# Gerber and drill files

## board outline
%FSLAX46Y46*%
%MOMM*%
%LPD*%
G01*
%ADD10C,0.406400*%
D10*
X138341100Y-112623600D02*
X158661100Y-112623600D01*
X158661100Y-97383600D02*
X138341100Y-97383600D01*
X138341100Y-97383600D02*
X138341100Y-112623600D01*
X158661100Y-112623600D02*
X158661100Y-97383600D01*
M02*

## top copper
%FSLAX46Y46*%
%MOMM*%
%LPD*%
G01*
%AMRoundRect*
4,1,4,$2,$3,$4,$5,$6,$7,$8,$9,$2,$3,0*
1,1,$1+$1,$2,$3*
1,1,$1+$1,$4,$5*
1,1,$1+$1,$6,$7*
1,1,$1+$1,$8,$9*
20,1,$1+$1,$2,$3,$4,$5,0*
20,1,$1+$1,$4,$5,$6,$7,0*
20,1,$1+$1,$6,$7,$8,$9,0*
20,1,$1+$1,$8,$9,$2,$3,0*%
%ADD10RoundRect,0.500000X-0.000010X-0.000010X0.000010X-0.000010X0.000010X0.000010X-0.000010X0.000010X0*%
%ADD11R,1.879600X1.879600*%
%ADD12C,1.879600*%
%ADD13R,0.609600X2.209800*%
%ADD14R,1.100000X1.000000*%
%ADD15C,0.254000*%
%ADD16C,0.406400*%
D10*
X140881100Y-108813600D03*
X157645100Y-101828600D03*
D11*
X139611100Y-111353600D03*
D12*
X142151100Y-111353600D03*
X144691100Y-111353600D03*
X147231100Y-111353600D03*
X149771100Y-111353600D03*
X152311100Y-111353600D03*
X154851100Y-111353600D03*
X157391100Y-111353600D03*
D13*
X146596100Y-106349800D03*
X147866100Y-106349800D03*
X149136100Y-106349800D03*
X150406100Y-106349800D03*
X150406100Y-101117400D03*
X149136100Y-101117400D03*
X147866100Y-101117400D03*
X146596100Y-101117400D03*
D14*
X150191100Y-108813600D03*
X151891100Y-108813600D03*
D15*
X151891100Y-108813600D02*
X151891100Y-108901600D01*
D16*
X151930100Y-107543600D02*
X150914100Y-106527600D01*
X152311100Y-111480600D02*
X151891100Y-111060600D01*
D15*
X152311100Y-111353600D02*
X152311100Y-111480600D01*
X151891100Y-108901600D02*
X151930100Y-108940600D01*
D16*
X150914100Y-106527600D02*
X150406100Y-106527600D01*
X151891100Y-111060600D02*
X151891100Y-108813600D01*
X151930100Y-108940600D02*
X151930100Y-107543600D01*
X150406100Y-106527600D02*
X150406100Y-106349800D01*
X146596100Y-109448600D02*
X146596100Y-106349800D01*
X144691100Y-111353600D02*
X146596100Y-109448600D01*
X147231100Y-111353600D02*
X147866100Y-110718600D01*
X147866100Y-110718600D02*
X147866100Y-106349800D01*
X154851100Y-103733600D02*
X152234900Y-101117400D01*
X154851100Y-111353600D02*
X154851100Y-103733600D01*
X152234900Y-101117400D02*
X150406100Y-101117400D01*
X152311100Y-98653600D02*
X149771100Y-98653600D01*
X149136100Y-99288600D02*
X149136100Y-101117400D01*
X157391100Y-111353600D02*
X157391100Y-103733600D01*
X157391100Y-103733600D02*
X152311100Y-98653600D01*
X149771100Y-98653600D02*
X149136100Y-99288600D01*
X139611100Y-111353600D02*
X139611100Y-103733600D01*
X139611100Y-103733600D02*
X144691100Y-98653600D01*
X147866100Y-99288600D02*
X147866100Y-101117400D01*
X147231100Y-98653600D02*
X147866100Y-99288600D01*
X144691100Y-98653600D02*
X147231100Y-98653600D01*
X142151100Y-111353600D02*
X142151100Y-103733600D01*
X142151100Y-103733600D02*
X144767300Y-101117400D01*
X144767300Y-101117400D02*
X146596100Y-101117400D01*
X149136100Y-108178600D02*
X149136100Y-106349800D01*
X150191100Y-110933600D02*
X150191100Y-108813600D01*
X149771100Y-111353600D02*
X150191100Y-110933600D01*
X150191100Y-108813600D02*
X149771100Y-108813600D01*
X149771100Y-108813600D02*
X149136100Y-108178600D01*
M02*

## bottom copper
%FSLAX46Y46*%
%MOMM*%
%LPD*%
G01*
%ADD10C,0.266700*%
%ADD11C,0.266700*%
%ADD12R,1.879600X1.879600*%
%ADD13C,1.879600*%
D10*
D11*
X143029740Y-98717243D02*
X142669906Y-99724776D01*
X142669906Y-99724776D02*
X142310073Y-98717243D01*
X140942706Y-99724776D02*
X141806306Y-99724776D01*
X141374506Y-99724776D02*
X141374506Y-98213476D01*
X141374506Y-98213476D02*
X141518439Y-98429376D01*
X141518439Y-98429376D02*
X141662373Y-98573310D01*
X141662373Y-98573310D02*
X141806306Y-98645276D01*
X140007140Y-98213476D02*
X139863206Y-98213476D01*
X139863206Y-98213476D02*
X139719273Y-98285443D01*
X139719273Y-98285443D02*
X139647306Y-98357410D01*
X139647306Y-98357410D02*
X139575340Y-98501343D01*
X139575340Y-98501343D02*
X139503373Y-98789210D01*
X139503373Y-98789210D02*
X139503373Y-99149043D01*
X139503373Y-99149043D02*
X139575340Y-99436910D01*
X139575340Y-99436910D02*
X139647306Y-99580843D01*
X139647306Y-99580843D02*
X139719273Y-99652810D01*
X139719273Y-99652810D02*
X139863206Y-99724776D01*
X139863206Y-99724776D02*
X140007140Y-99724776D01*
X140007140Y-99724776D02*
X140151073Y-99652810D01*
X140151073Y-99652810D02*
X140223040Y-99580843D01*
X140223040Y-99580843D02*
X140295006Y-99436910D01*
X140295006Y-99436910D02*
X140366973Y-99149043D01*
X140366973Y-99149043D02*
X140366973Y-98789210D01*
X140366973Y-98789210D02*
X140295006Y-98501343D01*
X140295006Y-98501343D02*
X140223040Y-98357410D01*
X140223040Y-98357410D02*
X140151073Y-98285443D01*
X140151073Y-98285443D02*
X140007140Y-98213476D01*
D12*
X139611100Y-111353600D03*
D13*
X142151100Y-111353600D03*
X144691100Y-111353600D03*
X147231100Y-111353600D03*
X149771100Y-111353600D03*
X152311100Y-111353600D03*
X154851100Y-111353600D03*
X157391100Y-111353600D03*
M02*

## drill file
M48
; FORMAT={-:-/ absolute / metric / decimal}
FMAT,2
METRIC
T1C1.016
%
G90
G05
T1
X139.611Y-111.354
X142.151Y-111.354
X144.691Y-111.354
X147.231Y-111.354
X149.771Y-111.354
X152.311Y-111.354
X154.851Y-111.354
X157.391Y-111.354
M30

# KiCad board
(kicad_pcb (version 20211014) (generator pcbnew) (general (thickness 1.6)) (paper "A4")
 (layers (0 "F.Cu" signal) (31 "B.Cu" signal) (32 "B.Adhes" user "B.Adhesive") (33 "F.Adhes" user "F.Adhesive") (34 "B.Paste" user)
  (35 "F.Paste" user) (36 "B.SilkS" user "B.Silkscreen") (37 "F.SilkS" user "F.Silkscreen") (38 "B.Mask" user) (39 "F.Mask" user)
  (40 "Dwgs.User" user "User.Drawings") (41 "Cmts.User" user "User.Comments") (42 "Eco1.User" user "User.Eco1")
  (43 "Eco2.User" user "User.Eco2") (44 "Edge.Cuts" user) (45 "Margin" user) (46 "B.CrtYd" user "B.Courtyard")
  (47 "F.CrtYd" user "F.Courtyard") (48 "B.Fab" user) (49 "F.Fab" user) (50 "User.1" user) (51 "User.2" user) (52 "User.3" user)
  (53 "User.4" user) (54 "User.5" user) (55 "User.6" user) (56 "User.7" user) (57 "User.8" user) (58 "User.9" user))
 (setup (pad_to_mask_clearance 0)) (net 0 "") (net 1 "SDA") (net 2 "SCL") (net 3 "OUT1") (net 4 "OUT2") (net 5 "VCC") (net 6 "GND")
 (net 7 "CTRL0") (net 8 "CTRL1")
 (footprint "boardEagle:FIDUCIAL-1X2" (layer "F.Cu") (at 140.8811 108.8136)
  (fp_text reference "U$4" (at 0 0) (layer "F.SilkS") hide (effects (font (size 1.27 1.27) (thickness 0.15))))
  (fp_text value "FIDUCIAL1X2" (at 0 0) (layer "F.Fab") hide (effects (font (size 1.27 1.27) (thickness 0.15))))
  (pad "1" smd roundrect (at 0 0) (size 1 1) (layers "F.Cu" "F.Mask") (roundrect_rratio 0.5) (solder_mask_margin 0.1016)))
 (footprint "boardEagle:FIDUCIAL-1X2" (layer "F.Cu") (at 157.6451 101.8286)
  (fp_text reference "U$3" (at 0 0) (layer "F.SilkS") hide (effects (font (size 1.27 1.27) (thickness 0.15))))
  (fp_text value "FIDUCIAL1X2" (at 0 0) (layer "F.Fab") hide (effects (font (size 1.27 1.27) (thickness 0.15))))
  (pad "1" smd roundrect (at 0 0) (size 1 1) (layers "F.Cu" "F.Mask") (roundrect_rratio 0.5) (solder_mask_margin 0.1016)))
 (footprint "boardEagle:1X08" (layer "F.Cu") (at 139.6111 111.3536)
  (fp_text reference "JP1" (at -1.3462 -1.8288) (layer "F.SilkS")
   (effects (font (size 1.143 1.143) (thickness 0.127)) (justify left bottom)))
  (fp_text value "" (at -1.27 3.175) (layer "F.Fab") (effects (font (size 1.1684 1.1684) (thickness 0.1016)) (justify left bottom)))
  (pad "1" thru_hole rect (at 0 0 90) (size 1.8796 1.8796) (drill 1.016) (layers *.Cu *.Mask) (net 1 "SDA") (solder_mask_margin 0.1016))
  (pad "2" thru_hole circle (at 2.54 0 90) (size 1.8796 1.8796) (drill 1.016) (layers *.Cu *.Mask) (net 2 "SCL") (solder_mask_margin 0.1016))
  (pad "3" thru_hole circle (at 5.08 0 90) (size 1.8796 1.8796) (drill 1.016) (layers *.Cu *.Mask) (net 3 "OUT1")
   (solder_mask_margin 0.1016))
  (pad "4" thru_hole circle (at 7.62 0 90) (size 1.8796 1.8796) (drill 1.016) (layers *.Cu *.Mask) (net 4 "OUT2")
   (solder_mask_margin 0.1016))
  (pad "5" thru_hole circle (at 10.16 0 90) (size 1.8796 1.8796) (drill 1.016) (layers *.Cu *.Mask) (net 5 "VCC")
   (solder_mask_margin 0.1016))
  (pad "6" thru_hole circle (at 12.7 0 90) (size 1.8796 1.8796) (drill 1.016) (layers *.Cu *.Mask) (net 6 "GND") (solder_mask_margin 0.1016))
  (pad "7" thru_hole circle (at 15.24 0 90) (size 1.8796 1.8796) (drill 1.016) (layers *.Cu *.Mask) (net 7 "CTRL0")
   (solder_mask_margin 0.1016))
  (pad "8" thru_hole circle (at 17.78 0 90) (size 1.8796 1.8796) (drill 1.016) (layers *.Cu *.Mask) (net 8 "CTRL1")
   (solder_mask_margin 0.1016)))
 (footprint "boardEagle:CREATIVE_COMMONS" (layer "F.Cu") (at 73.090088 112.6236)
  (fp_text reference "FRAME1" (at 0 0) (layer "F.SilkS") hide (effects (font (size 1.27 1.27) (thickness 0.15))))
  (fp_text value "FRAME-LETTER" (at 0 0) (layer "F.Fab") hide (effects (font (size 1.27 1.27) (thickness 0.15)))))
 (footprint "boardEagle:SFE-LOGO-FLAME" (layer "F.Cu") (at 139.6111 101.1936)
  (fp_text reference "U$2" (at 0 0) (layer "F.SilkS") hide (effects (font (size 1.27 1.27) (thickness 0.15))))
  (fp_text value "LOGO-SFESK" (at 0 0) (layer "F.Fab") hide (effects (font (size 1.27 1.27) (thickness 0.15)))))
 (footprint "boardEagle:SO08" (layer "F.Cu") (at 148.5011 103.7336)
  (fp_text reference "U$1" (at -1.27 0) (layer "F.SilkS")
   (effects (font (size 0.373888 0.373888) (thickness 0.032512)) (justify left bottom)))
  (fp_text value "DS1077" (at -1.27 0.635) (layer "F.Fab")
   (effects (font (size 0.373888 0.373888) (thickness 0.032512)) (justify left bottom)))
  (pad "1" smd rect (at -1.905 2.6162) (size 0.6096 2.2098) (layers "F.Cu" "F.Paste" "F.Mask") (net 3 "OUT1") (solder_mask_margin 0.1016))
  (pad "2" smd rect (at -0.635 2.6162) (size 0.6096 2.2098) (layers "F.Cu" "F.Paste" "F.Mask") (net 4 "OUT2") (solder_mask_margin 0.1016))
  (pad "3" smd rect (at 0.635 2.6162) (size 0.6096 2.2098) (layers "F.Cu" "F.Paste" "F.Mask") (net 5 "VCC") (solder_mask_margin 0.1016))
  (pad "4" smd rect (at 1.905 2.6162) (size 0.6096 2.2098) (layers "F.Cu" "F.Paste" "F.Mask") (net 6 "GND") (solder_mask_margin 0.1016))
  (pad "5" smd rect (at 1.905 -2.6162) (size 0.6096 2.2098) (layers "F.Cu" "F.Paste" "F.Mask") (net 7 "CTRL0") (solder_mask_margin 0.1016))
  (pad "6" smd rect (at 0.635 -2.6162) (size 0.6096 2.2098) (layers "F.Cu" "F.Paste" "F.Mask") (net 8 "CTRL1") (solder_mask_margin 0.1016))
  (pad "7" smd rect (at -0.635 -2.6162) (size 0.6096 2.2098) (layers "F.Cu" "F.Paste" "F.Mask") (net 1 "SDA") (solder_mask_margin 0.1016))
  (pad "8" smd rect (at -1.905 -2.6162) (size 0.6096 2.2098) (layers "F.Cu" "F.Paste" "F.Mask") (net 2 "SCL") (solder_mask_margin 0.1016)))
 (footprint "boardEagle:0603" (layer "F.Cu") (at 151.0411 108.8136)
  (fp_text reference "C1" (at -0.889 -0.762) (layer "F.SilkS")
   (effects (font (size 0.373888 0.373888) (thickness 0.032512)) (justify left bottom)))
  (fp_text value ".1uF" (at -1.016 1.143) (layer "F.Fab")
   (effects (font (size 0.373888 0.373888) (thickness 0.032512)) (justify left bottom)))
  (pad "1" smd rect (at -0.85 0) (size 1.1 1) (layers "F.Cu" "F.Paste" "F.Mask") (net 5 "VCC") (solder_mask_margin 0.1016))
  (pad "2" smd rect (at 0.85 0) (size 1.1 1) (layers "F.Cu" "F.Paste" "F.Mask") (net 6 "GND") (solder_mask_margin 0.1016)))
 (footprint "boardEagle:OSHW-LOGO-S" (layer "F.Cu") (at 156.6291 99.5426)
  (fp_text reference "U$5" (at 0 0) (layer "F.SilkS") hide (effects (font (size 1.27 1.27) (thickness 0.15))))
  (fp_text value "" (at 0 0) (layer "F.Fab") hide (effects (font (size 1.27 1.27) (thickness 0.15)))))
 (gr_line (start 138.3411 112.6236) (end 158.6611 112.6236) (layer "Edge.Cuts") (width 0.4064))
 (gr_line (start 158.6611 97.3836) (end 138.3411 97.3836) (layer "Edge.Cuts") (width 0.4064))
 (gr_line (start 138.3411 97.3836) (end 138.3411 112.6236) (layer "Edge.Cuts") (width 0.4064))
 (gr_line (start 158.6611 112.6236) (end 158.6611 97.3836) (layer "Edge.Cuts") (width 0.4064))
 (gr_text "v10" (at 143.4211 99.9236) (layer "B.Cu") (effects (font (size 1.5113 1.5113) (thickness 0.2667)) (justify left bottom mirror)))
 (segment (start 151.8911 108.8136) (end 151.8911 108.9016) (width 0.254) (layer "F.Cu") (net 6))
 (segment (start 151.9301 107.5436) (end 150.9141 106.5276) (width 0.4064) (layer "F.Cu") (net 6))
 (segment (start 152.3111 111.4806) (end 151.8911 111.0606) (width 0.4064) (layer "F.Cu") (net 6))
 (segment (start 152.3111 111.3536) (end 152.3111 111.4806) (width 0.254) (layer "F.Cu") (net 6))
 (segment (start 151.8911 108.9016) (end 151.9301 108.9406) (width 0.254) (layer "F.Cu") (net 6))
 (segment (start 150.9141 106.5276) (end 150.4061 106.5276) (width 0.4064) (layer "F.Cu") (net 6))
 (segment (start 151.8911 111.0606) (end 151.8911 108.8136) (width 0.4064) (layer "F.Cu") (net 6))
 (segment (start 151.9301 108.9406) (end 151.9301 107.5436) (width 0.4064) (layer "F.Cu") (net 6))
 (segment (start 150.4061 106.5276) (end 150.4061 106.3498) (width 0.4064) (layer "F.Cu") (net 6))
 (segment (start 146.5961 109.4486) (end 146.5961 106.3498) (width 0.4064) (layer "F.Cu") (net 3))
 (segment (start 144.6911 111.3536) (end 146.5961 109.4486) (width 0.4064) (layer "F.Cu") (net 3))
 (segment (start 147.2311 111.3536) (end 147.8661 110.7186) (width 0.4064) (layer "F.Cu") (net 4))
 (segment (start 147.8661 110.7186) (end 147.8661 106.3498) (width 0.4064) (layer "F.Cu") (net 4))
 (segment (start 154.8511 103.7336) (end 152.2349 101.1174) (width 0.4064) (layer "F.Cu") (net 7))
 (segment (start 154.8511 111.3536) (end 154.8511 103.7336) (width 0.4064) (layer "F.Cu") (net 7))
 (segment (start 152.2349 101.1174) (end 150.4061 101.1174) (width 0.4064) (layer "F.Cu") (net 7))
 (segment (start 152.3111 98.6536) (end 149.7711 98.6536) (width 0.4064) (layer "F.Cu") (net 8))
 (segment (start 149.1361 99.2886) (end 149.1361 101.1174) (width 0.4064) (layer "F.Cu") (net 8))
 (segment (start 157.3911 111.3536) (end 157.3911 103.7336) (width 0.4064) (layer "F.Cu") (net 8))
 (segment (start 157.3911 103.7336) (end 152.3111 98.6536) (width 0.4064) (layer "F.Cu") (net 8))
 (segment (start 149.7711 98.6536) (end 149.1361 99.2886) (width 0.4064) (layer "F.Cu") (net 8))
 (segment (start 139.6111 111.3536) (end 139.6111 103.7336) (width 0.4064) (layer "F.Cu") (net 1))
 (segment (start 139.6111 103.7336) (end 144.6911 98.6536) (width 0.4064) (layer "F.Cu") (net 1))
 (segment (start 147.8661 99.2886) (end 147.8661 101.1174) (width 0.4064) (layer "F.Cu") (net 1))
 (segment (start 147.2311 98.6536) (end 147.8661 99.2886) (width 0.4064) (layer "F.Cu") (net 1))
 (segment (start 144.6911 98.6536) (end 147.2311 98.6536) (width 0.4064) (layer "F.Cu") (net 1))
 (segment (start 142.1511 111.3536) (end 142.1511 103.7336) (width 0.4064) (layer "F.Cu") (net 2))
 (segment (start 142.1511 103.7336) (end 144.7673 101.1174) (width 0.4064) (layer "F.Cu") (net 2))
 (segment (start 144.7673 101.1174) (end 146.5961 101.1174) (width 0.4064) (layer "F.Cu") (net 2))
 (segment (start 149.1361 108.1786) (end 149.1361 106.3498) (width 0.4064) (layer "F.Cu") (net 5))
 (segment (start 150.1911 110.9336) (end 150.1911 108.8136) (width 0.4064) (layer "F.Cu") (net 5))
 (segment (start 149.7711 111.3536) (end 150.1911 110.9336) (width 0.4064) (layer "F.Cu") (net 5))
 (segment (start 150.1911 108.8136) (end 149.7711 108.8136) (width 0.4064) (layer "F.Cu") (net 5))
 (segment (start 149.7711 108.8136) (end 149.1361 108.1786) (width 0.4064) (layer "F.Cu") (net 5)))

